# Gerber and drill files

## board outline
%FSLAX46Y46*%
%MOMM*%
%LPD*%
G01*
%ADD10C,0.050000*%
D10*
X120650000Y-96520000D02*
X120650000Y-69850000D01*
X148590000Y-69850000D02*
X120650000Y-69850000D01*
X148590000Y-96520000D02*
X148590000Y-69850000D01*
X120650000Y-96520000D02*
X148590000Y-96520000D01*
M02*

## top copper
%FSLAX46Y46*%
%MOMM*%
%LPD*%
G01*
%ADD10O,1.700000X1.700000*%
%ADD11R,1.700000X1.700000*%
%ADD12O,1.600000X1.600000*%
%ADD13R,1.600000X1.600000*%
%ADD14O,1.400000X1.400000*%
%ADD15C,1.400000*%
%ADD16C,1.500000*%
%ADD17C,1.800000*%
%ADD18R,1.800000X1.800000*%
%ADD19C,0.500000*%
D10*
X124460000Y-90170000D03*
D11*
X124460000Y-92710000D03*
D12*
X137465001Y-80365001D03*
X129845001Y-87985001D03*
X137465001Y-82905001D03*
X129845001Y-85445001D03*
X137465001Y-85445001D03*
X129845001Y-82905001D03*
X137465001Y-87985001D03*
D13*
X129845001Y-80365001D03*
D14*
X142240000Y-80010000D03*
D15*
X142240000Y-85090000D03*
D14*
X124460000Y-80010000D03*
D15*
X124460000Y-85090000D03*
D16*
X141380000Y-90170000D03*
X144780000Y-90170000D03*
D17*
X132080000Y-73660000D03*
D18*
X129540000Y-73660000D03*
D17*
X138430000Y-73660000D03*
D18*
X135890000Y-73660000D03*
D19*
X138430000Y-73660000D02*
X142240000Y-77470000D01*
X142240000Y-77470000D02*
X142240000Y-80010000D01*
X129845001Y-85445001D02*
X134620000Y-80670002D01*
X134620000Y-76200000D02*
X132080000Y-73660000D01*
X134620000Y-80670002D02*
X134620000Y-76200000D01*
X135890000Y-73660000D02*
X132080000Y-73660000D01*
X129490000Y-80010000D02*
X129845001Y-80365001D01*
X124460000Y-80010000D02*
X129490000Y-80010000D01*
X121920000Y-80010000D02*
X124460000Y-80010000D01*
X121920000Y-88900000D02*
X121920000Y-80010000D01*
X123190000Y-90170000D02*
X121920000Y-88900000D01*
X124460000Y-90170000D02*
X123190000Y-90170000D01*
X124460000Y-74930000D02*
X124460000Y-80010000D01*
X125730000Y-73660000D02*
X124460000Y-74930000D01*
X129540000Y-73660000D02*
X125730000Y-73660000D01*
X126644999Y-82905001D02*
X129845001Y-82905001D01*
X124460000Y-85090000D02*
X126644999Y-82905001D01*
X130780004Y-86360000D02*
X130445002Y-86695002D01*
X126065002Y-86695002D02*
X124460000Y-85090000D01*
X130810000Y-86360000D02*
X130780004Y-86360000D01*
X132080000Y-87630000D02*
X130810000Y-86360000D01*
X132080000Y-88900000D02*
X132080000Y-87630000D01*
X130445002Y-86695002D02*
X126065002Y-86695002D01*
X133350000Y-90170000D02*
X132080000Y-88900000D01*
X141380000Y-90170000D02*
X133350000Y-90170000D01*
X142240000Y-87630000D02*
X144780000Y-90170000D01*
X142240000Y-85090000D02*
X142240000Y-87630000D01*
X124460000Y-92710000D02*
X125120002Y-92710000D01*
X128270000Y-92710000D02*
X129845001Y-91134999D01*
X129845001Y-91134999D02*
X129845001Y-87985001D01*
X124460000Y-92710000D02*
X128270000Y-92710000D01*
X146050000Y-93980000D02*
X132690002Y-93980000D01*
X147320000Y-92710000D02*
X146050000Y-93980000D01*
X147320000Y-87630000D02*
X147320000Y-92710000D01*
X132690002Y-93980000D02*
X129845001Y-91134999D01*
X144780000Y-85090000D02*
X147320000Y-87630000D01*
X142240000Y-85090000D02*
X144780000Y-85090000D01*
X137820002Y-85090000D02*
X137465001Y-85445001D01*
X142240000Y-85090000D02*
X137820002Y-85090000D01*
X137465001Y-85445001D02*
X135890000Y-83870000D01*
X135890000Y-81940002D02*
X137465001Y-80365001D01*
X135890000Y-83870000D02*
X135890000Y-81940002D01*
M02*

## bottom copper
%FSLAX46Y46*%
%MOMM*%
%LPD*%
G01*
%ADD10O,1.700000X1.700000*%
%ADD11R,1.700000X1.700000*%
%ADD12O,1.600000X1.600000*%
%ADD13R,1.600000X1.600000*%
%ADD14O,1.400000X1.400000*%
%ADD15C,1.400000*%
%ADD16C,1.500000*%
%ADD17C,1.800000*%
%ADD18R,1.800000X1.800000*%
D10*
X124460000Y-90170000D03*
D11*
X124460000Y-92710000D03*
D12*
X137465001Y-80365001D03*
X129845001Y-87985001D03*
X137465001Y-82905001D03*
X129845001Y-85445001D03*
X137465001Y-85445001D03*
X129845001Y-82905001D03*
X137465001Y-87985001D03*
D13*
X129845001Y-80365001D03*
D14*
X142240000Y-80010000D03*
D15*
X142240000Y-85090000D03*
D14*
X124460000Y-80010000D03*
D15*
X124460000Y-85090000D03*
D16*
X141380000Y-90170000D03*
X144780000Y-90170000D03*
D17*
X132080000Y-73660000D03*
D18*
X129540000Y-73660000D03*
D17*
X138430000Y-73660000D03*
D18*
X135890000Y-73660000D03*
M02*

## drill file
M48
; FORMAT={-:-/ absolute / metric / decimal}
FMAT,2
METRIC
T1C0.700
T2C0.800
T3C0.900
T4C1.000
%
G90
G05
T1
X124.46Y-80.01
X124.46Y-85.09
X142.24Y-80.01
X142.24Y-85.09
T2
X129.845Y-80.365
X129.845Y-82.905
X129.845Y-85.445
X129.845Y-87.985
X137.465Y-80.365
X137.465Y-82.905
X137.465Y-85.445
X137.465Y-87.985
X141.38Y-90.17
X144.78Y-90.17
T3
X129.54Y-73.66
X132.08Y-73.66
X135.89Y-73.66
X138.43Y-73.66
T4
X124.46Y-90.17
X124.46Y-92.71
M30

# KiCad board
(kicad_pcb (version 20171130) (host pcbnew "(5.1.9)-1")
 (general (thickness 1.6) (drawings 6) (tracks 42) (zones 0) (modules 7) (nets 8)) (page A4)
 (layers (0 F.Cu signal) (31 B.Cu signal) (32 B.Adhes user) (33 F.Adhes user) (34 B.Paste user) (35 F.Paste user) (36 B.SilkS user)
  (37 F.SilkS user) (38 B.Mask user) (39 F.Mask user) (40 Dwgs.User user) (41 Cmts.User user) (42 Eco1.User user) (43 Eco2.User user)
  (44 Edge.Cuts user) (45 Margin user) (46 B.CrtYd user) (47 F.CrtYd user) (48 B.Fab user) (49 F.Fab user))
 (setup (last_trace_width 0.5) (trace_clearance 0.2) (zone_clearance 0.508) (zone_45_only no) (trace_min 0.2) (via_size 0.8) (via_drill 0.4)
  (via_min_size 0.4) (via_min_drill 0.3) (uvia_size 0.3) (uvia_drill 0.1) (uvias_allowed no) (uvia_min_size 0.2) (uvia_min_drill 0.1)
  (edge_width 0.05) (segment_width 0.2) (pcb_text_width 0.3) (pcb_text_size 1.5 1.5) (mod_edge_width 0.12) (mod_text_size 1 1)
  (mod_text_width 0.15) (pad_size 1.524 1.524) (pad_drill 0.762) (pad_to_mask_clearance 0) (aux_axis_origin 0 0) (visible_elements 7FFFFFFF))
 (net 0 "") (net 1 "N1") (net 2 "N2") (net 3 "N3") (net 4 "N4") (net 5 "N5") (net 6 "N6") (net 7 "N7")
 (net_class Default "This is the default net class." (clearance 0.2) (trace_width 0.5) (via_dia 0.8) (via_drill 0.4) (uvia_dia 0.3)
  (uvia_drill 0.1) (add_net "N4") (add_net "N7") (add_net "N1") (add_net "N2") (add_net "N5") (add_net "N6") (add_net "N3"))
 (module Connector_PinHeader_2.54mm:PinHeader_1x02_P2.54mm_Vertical (layer F.Cu) (at 124.46 92.71 180)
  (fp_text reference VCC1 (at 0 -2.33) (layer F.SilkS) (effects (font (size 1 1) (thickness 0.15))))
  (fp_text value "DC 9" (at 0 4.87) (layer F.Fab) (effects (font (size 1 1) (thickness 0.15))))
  (pad 2 thru_hole oval (at 0 2.54 180) (size 1.7 1.7) (drill 1) (layers *.Cu *.Mask) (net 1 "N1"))
  (pad 1 thru_hole rect (at 0 0 180) (size 1.7 1.7) (drill 1) (layers *.Cu *.Mask) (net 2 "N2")))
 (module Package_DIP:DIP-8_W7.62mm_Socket (layer F.Cu) (at 129.845001 80.365001)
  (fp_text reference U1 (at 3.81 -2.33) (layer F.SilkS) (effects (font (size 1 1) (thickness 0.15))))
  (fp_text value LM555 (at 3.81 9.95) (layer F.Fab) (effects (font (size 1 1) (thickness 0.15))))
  (pad 8 thru_hole oval (at 7.62 0) (size 1.6 1.6) (drill 0.8) (layers *.Cu *.Mask) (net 2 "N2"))
  (pad 4 thru_hole oval (at 0 7.62) (size 1.6 1.6) (drill 0.8) (layers *.Cu *.Mask) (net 2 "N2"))
  (pad 7 thru_hole oval (at 7.62 2.54) (size 1.6 1.6) (drill 0.8) (layers *.Cu *.Mask) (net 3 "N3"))
  (pad 3 thru_hole oval (at 0 5.08) (size 1.6 1.6) (drill 0.8) (layers *.Cu *.Mask) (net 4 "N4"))
  (pad 6 thru_hole oval (at 7.62 5.08) (size 1.6 1.6) (drill 0.8) (layers *.Cu *.Mask) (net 2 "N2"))
  (pad 2 thru_hole oval (at 0 2.54) (size 1.6 1.6) (drill 0.8) (layers *.Cu *.Mask) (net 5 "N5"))
  (pad 5 thru_hole oval (at 7.62 7.62) (size 1.6 1.6) (drill 0.8) (layers *.Cu *.Mask) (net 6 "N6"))
  (pad 1 thru_hole rect (at 0 0) (size 1.6 1.6) (drill 0.8) (layers *.Cu *.Mask) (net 1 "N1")))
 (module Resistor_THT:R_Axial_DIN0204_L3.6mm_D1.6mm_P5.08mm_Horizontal (layer F.Cu) (at 142.24 85.09 90)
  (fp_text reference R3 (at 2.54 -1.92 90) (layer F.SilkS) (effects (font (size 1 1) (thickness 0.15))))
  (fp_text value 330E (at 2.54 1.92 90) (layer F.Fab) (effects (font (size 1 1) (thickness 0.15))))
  (pad 2 thru_hole oval (at 5.08 0 90) (size 1.4 1.4) (drill 0.7) (layers *.Cu *.Mask) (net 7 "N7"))
  (pad 1 thru_hole circle (at 0 0 90) (size 1.4 1.4) (drill 0.7) (layers *.Cu *.Mask) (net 2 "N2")))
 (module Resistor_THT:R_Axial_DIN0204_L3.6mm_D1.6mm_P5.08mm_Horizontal (layer F.Cu) (at 124.46 85.09 90)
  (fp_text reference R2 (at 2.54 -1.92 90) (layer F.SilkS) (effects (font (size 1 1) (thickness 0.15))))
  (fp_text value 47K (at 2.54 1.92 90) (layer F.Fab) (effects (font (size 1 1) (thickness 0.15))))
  (pad 2 thru_hole oval (at 5.08 0 90) (size 1.4 1.4) (drill 0.7) (layers *.Cu *.Mask) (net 1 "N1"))
  (pad 1 thru_hole circle (at 0 0 90) (size 1.4 1.4) (drill 0.7) (layers *.Cu *.Mask) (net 5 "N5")))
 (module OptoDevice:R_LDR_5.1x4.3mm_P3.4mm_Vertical (layer F.Cu) (at 144.78 90.17 180)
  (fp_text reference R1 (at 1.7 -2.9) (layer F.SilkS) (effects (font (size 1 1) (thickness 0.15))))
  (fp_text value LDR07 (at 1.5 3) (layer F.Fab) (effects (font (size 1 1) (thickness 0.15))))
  (pad 2 thru_hole circle (at 3.4 0 180) (size 1.5 1.5) (drill 0.8) (layers *.Cu *.Mask) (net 5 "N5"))
  (pad 1 thru_hole circle (at 0 0 180) (size 1.5 1.5) (drill 0.8) (layers *.Cu *.Mask) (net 2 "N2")))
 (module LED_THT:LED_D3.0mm (layer F.Cu) (at 129.54 73.66)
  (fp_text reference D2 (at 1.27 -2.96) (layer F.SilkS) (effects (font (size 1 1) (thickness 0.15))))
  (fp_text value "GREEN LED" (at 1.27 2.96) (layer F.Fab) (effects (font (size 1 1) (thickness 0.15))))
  (pad 2 thru_hole circle (at 2.54 0) (size 1.8 1.8) (drill 0.9) (layers *.Cu *.Mask) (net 4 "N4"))
  (pad 1 thru_hole rect (at 0 0) (size 1.8 1.8) (drill 0.9) (layers *.Cu *.Mask) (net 1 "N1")))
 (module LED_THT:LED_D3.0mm (layer F.Cu) (at 135.89 73.66)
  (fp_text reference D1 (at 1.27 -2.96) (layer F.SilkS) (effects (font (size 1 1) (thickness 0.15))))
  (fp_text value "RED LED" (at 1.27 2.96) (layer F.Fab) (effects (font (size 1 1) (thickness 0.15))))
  (pad 2 thru_hole circle (at 2.54 0) (size 1.8 1.8) (drill 0.9) (layers *.Cu *.Mask) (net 7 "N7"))
  (pad 1 thru_hole rect (at 0 0) (size 1.8 1.8) (drill 0.9) (layers *.Cu *.Mask) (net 4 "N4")))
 (gr_line (start 120.65 96.52) (end 120.65 69.85) (layer Edge.Cuts) (width 0.05))
 (gr_line (start 148.59 69.85) (end 120.65 69.85) (layer Edge.Cuts) (width 0.05))
 (gr_line (start 148.59 96.52) (end 148.59 69.85) (layer Edge.Cuts) (width 0.05))
 (gr_line (start 120.65 96.52) (end 148.59 96.52) (layer Edge.Cuts) (width 0.05))
 (segment (start 138.43 73.66) (end 142.24 77.47) (width 0.5) (layer F.Cu) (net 7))
 (segment (start 142.24 77.47) (end 142.24 80.01) (width 0.5) (layer F.Cu) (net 7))
 (segment (start 129.845001 85.445001) (end 134.62 80.670002) (width 0.5) (layer F.Cu) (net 4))
 (segment (start 134.62 76.2) (end 132.08 73.66) (width 0.5) (layer F.Cu) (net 4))
 (segment (start 134.62 80.670002) (end 134.62 76.2) (width 0.5) (layer F.Cu) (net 4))
 (segment (start 135.89 73.66) (end 132.08 73.66) (width 0.5) (layer F.Cu) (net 4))
 (segment (start 129.49 80.01) (end 129.845001 80.365001) (width 0.5) (layer F.Cu) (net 1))
 (segment (start 124.46 80.01) (end 129.49 80.01) (width 0.5) (layer F.Cu) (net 1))
 (segment (start 121.92 80.01) (end 124.46 80.01) (width 0.5) (layer F.Cu) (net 1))
 (segment (start 121.92 88.9) (end 121.92 80.01) (width 0.5) (layer F.Cu) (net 1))
 (segment (start 123.19 90.17) (end 121.92 88.9) (width 0.5) (layer F.Cu) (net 1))
 (segment (start 124.46 90.17) (end 123.19 90.17) (width 0.5) (layer F.Cu) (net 1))
 (segment (start 124.46 74.93) (end 124.46 80.01) (width 0.5) (layer F.Cu) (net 1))
 (segment (start 125.73 73.66) (end 124.46 74.93) (width 0.5) (layer F.Cu) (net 1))
 (segment (start 129.54 73.66) (end 125.73 73.66) (width 0.5) (layer F.Cu) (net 1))
 (segment (start 126.644999 82.905001) (end 129.845001 82.905001) (width 0.5) (layer F.Cu) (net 5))
 (segment (start 124.46 85.09) (end 126.644999 82.905001) (width 0.5) (layer F.Cu) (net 5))
 (segment (start 130.780004 86.36) (end 130.445002 86.695002) (width 0.5) (layer F.Cu) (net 5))
 (segment (start 126.065002 86.695002) (end 124.46 85.09) (width 0.5) (layer F.Cu) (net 5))
 (segment (start 130.81 86.36) (end 130.780004 86.36) (width 0.5) (layer F.Cu) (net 5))
 (segment (start 132.08 87.63) (end 130.81 86.36) (width 0.5) (layer F.Cu) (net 5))
 (segment (start 132.08 88.9) (end 132.08 87.63) (width 0.5) (layer F.Cu) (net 5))
 (segment (start 130.445002 86.695002) (end 126.065002 86.695002) (width 0.5) (layer F.Cu) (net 5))
 (segment (start 133.35 90.17) (end 132.08 88.9) (width 0.5) (layer F.Cu) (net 5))
 (segment (start 141.38 90.17) (end 133.35 90.17) (width 0.5) (layer F.Cu) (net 5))
 (segment (start 142.24 87.63) (end 144.78 90.17) (width 0.5) (layer F.Cu) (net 2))
 (segment (start 142.24 85.09) (end 142.24 87.63) (width 0.5) (layer F.Cu) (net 2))
 (segment (start 124.46 92.71) (end 125.120002 92.71) (width 0.5) (layer F.Cu) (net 2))
 (segment (start 128.27 92.71) (end 129.845001 91.134999) (width 0.5) (layer F.Cu) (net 2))
 (segment (start 129.845001 91.134999) (end 129.845001 87.985001) (width 0.5) (layer F.Cu) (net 2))
 (segment (start 124.46 92.71) (end 128.27 92.71) (width 0.5) (layer F.Cu) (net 2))
 (segment (start 146.05 93.98) (end 132.690002 93.98) (width 0.5) (layer F.Cu) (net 2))
 (segment (start 147.32 92.71) (end 146.05 93.98) (width 0.5) (layer F.Cu) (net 2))
 (segment (start 147.32 87.63) (end 147.32 92.71) (width 0.5) (layer F.Cu) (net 2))
 (segment (start 132.690002 93.98) (end 129.845001 91.134999) (width 0.5) (layer F.Cu) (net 2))
 (segment (start 144.78 85.09) (end 147.32 87.63) (width 0.5) (layer F.Cu) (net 2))
 (segment (start 142.24 85.09) (end 144.78 85.09) (width 0.5) (layer F.Cu) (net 2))
 (segment (start 137.820002 85.09) (end 137.465001 85.445001) (width 0.5) (layer F.Cu) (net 2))
 (segment (start 142.24 85.09) (end 137.820002 85.09) (width 0.5) (layer F.Cu) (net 2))
 (segment (start 137.465001 85.445001) (end 135.89 83.87) (width 0.5) (layer F.Cu) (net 2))
 (segment (start 135.89 81.940002) (end 137.465001 80.365001) (width 0.5) (layer F.Cu) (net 2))
 (segment (start 135.89 83.87) (end 135.89 81.940002) (width 0.5) (layer F.Cu) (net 2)))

